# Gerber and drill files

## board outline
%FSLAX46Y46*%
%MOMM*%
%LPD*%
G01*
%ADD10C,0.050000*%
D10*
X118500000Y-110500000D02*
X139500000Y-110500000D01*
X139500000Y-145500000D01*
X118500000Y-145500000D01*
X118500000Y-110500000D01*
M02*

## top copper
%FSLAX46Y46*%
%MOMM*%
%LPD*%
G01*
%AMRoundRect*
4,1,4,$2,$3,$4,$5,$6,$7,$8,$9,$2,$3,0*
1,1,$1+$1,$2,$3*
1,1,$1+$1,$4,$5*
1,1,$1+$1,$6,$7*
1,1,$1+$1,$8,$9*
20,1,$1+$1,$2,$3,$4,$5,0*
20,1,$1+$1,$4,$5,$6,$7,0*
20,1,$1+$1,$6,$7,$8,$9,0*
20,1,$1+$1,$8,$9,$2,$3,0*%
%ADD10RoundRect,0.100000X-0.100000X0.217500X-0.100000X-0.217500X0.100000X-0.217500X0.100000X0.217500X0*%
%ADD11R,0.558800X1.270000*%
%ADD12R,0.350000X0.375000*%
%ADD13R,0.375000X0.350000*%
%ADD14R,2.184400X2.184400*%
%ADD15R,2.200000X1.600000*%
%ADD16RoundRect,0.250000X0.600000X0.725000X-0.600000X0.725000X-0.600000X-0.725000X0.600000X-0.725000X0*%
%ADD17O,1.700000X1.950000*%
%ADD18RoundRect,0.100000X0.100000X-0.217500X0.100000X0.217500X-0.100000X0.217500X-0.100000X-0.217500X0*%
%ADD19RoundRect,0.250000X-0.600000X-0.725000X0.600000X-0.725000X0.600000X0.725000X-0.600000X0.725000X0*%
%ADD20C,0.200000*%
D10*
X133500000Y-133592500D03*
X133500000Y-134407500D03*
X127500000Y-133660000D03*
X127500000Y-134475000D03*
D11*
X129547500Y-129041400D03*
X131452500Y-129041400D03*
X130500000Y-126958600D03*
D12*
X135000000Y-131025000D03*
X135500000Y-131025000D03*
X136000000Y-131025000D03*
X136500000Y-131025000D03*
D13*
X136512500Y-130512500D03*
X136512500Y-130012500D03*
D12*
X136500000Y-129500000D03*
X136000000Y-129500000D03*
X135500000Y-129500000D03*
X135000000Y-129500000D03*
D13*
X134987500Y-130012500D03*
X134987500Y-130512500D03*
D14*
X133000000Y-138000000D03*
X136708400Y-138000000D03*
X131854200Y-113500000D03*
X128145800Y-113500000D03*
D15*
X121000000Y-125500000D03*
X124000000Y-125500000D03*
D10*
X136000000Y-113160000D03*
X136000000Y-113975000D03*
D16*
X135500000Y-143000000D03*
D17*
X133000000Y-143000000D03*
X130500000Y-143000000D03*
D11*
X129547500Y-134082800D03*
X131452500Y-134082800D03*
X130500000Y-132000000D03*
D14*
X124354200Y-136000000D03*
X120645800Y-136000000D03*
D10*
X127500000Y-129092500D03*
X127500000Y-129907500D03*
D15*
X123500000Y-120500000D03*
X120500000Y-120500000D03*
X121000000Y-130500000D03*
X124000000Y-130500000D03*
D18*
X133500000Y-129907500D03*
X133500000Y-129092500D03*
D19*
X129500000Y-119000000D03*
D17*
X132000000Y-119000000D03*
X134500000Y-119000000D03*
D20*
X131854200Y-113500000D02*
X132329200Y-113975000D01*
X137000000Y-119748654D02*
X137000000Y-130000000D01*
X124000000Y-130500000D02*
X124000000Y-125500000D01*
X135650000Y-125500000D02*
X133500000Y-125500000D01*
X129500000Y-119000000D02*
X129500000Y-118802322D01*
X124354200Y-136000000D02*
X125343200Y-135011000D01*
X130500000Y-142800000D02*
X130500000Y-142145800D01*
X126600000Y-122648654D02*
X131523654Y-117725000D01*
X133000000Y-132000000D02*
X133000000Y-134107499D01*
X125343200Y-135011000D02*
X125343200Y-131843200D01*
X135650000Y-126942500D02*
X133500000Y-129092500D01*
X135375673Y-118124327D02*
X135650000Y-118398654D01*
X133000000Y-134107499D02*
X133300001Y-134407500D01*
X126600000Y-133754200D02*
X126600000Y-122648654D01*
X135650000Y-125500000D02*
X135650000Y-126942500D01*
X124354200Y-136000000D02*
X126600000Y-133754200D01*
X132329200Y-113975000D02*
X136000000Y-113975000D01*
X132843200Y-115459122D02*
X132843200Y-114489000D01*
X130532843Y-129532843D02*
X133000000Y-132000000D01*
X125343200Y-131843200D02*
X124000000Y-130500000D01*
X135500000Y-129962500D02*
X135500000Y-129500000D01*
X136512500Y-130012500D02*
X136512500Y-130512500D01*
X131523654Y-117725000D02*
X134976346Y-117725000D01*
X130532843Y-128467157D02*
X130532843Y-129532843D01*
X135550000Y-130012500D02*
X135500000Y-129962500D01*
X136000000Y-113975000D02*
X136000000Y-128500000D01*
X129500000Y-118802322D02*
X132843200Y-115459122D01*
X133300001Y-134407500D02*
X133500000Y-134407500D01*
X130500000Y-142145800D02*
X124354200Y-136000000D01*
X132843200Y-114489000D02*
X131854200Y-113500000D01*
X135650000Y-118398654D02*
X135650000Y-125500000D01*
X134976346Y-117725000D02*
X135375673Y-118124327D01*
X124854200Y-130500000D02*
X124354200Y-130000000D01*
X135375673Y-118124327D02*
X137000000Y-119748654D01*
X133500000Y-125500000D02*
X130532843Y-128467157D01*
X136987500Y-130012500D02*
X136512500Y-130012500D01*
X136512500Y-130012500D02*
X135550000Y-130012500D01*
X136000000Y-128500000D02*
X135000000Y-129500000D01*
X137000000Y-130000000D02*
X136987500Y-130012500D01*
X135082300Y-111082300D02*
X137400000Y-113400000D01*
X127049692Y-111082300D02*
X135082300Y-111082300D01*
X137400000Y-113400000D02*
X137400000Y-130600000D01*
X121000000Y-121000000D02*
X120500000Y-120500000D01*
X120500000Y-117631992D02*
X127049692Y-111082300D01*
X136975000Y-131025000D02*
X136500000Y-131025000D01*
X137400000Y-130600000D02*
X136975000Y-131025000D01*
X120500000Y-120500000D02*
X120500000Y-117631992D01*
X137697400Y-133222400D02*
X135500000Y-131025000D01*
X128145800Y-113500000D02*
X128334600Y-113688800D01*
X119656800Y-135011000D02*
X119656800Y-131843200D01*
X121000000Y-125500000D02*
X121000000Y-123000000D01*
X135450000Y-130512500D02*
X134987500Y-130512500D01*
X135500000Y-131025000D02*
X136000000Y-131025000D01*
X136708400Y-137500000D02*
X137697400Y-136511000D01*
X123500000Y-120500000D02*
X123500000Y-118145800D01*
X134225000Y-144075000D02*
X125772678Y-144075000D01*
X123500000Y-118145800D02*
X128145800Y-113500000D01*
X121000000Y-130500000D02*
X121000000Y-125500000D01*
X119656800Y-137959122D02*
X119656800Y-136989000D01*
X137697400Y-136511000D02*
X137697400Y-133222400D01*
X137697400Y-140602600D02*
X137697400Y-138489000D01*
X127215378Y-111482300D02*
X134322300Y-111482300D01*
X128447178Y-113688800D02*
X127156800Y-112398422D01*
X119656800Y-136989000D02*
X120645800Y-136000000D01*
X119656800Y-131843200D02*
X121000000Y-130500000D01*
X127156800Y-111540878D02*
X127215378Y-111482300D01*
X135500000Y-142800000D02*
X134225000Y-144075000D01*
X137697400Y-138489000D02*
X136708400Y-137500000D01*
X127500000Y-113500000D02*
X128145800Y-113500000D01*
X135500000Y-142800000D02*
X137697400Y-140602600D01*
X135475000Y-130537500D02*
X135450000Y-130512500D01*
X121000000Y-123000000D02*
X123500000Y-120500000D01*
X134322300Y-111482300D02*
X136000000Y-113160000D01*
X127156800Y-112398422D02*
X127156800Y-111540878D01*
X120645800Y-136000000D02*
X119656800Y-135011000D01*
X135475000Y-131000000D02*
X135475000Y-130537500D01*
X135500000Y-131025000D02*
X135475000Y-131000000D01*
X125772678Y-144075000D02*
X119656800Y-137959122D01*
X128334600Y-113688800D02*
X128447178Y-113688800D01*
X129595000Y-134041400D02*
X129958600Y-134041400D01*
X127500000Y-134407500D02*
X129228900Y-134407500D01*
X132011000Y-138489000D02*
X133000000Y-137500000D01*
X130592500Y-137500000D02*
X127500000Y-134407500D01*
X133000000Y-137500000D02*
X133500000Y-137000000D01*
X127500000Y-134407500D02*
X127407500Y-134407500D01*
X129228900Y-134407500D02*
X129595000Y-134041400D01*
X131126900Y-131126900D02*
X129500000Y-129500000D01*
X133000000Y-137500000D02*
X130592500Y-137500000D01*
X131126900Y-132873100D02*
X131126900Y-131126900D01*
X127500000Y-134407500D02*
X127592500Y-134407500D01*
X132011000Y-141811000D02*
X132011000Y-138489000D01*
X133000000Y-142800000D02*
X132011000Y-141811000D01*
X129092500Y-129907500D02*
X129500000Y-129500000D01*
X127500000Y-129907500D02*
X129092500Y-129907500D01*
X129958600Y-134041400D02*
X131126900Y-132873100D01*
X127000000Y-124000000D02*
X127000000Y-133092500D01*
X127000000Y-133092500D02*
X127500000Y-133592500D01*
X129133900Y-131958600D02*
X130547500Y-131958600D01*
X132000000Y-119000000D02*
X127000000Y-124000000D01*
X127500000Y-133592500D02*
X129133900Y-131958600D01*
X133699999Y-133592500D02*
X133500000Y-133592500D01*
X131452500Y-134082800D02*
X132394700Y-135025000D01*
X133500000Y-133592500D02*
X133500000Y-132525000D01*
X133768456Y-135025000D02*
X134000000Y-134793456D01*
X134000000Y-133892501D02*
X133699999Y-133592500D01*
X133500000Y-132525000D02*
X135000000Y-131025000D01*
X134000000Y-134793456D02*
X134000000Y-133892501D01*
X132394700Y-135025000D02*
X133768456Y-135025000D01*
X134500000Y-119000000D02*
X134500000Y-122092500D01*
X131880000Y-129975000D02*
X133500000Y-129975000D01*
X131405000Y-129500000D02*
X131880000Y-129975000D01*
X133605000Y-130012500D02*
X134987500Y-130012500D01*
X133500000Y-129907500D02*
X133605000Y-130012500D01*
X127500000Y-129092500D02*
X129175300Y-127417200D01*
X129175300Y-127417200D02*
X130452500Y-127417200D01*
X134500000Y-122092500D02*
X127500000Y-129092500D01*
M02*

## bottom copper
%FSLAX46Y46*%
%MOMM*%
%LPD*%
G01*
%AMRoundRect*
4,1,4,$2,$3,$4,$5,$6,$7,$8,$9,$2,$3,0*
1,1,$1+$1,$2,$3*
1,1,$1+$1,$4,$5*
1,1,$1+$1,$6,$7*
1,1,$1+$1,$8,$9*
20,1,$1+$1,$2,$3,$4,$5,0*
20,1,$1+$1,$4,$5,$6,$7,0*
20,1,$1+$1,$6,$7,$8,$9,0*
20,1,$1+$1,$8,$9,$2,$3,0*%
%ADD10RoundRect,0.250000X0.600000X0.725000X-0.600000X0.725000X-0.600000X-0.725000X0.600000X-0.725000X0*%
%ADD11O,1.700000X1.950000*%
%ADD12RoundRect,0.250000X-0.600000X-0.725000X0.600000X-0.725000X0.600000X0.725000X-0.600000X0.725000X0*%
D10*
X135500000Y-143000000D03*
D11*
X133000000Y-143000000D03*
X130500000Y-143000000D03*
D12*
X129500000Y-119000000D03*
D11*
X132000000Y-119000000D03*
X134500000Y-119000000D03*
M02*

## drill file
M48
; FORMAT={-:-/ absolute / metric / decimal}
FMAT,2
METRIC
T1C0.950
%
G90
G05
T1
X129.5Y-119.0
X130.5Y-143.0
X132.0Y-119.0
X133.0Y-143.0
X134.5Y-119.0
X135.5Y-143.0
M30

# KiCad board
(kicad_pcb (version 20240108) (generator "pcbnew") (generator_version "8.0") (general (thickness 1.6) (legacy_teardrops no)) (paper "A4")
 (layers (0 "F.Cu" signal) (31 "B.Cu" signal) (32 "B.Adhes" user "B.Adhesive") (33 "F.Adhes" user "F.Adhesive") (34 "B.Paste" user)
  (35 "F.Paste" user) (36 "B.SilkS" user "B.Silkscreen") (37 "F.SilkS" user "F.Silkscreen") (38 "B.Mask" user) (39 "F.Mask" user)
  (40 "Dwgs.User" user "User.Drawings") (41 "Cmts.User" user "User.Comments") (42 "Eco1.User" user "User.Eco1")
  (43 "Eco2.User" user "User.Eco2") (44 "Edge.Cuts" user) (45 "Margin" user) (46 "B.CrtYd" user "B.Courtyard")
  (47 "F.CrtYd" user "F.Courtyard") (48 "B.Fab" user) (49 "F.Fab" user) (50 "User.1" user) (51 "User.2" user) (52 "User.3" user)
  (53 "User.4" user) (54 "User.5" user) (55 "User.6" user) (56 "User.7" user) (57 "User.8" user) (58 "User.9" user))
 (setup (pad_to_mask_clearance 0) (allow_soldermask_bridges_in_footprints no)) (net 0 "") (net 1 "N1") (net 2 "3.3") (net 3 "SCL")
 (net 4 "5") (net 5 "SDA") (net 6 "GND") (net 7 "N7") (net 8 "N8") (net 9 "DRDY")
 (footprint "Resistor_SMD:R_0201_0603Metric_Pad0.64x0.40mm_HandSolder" (layer "F.Cu") (at 133.5 134 -90)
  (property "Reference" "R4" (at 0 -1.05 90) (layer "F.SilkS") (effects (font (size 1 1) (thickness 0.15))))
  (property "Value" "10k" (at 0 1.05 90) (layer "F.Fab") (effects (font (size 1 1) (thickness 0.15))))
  (pad "" smd roundrect (at -0.4325 0 270) (size 0.458 0.36) (layers "F.Paste") (roundrect_rratio 0.25))
  (pad "" smd roundrect (at 0.4325 0 270) (size 0.458 0.36) (layers "F.Paste") (roundrect_rratio 0.25))
  (pad "1" smd roundrect (at -0.4075 0 270) (size 0.635 0.4) (layers "F.Cu" "F.Mask") (roundrect_rratio 0.25) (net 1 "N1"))
  (pad "2" smd roundrect (at 0.4075 0 270) (size 0.635 0.4) (layers "F.Cu" "F.Mask") (roundrect_rratio 0.25) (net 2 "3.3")))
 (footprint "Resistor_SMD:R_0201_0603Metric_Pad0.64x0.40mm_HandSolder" (layer "F.Cu") (at 127.5 134.0675 -90)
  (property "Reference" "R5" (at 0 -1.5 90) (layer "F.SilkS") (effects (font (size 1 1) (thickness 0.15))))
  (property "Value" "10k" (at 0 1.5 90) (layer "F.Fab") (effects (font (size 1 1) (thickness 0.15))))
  (pad "" smd roundrect (at -0.4325 0 270) (size 0.458 0.36) (layers "F.Paste") (roundrect_rratio 0.25))
  (pad "" smd roundrect (at 0.4325 0 270) (size 0.458 0.36) (layers "F.Paste") (roundrect_rratio 0.25))
  (pad "1" smd roundrect (at -0.4075 0 270) (size 0.635 0.4) (layers "F.Cu" "F.Mask") (roundrect_rratio 0.25) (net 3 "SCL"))
  (pad "2" smd roundrect (at 0.4075 0 270) (size 0.635 0.4) (layers "F.Cu" "F.Mask") (roundrect_rratio 0.25) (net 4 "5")))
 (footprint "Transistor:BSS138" (layer "F.Cu") (at 130.5 128)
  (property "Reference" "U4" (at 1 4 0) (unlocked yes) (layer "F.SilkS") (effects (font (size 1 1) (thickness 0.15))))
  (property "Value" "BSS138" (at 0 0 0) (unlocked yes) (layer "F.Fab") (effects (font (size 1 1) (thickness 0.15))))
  (pad "1" smd rect (at -0.9525 1.0414) (size 0.5588 1.27) (layers "F.Cu" "F.Paste" "F.Mask") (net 4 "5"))
  (pad "2" smd rect (at 0.9525 1.0414) (size 0.5588 1.27) (layers "F.Cu" "F.Paste" "F.Mask") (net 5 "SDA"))
  (pad "3" smd rect (at 0 -1.0414) (size 0.5588 1.27) (layers "F.Cu" "F.Paste" "F.Mask") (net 5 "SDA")))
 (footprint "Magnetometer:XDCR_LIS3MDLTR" (layer "F.Cu") (at 135.75 130.2625 90)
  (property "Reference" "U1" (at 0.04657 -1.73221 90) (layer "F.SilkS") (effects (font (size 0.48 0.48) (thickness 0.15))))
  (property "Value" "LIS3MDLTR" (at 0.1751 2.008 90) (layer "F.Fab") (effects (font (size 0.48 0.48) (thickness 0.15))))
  (pad "1" smd rect (at -0.7625 -0.75 90) (size 0.375 0.35) (layers "F.Cu" "F.Paste") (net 1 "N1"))
  (pad "2" smd rect (at -0.7625 -0.25 90) (size 0.375 0.35) (layers "F.Cu" "F.Paste") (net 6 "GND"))
  (pad "3" smd rect (at -0.7625 0.25 90) (size 0.375 0.35) (layers "F.Cu" "F.Paste") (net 6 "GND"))
  (pad "4" smd rect (at -0.7625 0.75 90) (size 0.375 0.35) (layers "F.Cu" "F.Paste") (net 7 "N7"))
  (pad "5" smd rect (at -0.25 0.7625 90) (size 0.35 0.375) (layers "F.Cu" "F.Paste") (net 2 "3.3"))
  (pad "6" smd rect (at 0.25 0.7625 90) (size 0.35 0.375) (layers "F.Cu" "F.Paste") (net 2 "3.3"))
  (pad "7" smd rect (at 0.7625 0.75 90) (size 0.375 0.35) (layers "F.Cu" "F.Paste") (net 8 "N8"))
  (pad "8" smd rect (at 0.7625 0.25 90) (size 0.375 0.35) (layers "F.Cu" "F.Paste") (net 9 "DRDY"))
  (pad "9" smd rect (at 0.7625 -0.25 90) (size 0.375 0.35) (layers "F.Cu" "F.Paste") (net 2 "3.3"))
  (pad "10" smd rect (at 0.7625 -0.75 90) (size 0.375 0.35) (layers "F.Cu" "F.Paste") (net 2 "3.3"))
  (pad "11" smd rect (at 0.25 -0.7625 90) (size 0.35 0.375) (layers "F.Cu" "F.Paste") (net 5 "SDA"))
  (pad "12" smd rect (at -0.25 -0.7625 90) (size 0.35 0.375) (layers "F.Cu" "F.Paste") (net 6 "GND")))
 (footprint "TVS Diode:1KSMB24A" (layer "F.Cu") (at 134.8542 138)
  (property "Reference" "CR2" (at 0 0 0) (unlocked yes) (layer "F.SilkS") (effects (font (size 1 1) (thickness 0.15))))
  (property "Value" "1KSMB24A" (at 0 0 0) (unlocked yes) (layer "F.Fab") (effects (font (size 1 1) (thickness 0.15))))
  (pad "1" smd rect (at -1.8542 0 90) (size 2.1844 2.1844) (layers "F.Cu" "F.Paste" "F.Mask") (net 4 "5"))
  (pad "2" smd rect (at 1.8542 0 90) (size 2.1844 2.1844) (layers "F.Cu" "F.Paste" "F.Mask") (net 6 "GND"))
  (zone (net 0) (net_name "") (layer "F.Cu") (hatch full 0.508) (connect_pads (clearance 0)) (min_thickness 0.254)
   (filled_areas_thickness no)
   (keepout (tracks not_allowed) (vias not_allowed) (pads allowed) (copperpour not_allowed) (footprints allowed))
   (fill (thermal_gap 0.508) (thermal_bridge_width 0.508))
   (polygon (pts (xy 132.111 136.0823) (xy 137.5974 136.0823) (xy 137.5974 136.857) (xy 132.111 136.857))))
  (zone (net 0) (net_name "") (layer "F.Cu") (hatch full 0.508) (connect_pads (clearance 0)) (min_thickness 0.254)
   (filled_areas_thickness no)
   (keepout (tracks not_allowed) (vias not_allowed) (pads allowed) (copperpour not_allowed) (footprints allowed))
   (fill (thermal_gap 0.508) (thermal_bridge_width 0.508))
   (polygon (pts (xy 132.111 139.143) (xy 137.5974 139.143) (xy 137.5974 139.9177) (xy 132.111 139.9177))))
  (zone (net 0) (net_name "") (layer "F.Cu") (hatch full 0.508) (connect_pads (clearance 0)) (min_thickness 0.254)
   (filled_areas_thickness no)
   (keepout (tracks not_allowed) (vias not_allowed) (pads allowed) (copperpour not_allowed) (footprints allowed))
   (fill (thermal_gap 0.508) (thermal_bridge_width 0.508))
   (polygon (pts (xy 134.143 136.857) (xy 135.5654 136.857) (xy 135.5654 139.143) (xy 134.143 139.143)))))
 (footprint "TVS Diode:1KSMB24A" (layer "F.Cu") (at 130 113.5 180)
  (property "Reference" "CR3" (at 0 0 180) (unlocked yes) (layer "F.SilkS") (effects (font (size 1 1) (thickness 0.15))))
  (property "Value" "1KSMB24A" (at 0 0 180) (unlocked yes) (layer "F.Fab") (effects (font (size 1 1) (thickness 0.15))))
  (pad "1" smd rect (at -1.8542 0 270) (size 2.1844 2.1844) (layers "F.Cu" "F.Paste" "F.Mask") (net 2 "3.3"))
  (pad "2" smd rect (at 1.8542 0 270) (size 2.1844 2.1844) (layers "F.Cu" "F.Paste" "F.Mask") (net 6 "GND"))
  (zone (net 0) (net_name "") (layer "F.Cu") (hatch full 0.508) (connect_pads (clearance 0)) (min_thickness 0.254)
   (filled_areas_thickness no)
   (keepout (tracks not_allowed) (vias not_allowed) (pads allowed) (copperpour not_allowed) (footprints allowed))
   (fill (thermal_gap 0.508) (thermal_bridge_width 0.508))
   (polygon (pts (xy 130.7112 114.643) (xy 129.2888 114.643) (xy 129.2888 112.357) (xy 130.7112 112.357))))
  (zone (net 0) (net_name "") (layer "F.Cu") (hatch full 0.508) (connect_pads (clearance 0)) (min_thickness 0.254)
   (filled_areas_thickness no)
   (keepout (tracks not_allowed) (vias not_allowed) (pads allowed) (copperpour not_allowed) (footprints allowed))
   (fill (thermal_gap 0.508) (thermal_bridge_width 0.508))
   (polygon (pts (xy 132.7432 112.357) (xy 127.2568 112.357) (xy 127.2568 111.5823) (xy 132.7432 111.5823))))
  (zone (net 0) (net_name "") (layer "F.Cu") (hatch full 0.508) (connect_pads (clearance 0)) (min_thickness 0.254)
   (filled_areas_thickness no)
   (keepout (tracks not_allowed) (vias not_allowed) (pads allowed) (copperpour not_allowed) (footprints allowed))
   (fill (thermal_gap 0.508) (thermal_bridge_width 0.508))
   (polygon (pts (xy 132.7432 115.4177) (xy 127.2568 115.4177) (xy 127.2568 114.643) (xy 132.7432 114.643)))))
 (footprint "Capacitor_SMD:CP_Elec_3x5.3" (layer "F.Cu") (at 122.5 125.5)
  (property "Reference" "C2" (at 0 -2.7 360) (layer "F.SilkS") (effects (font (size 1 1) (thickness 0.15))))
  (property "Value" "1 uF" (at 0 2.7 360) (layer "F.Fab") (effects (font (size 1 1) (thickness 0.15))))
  (pad "1" smd rect (at -1.5 0) (size 2.2 1.6) (layers "F.Cu" "F.Paste" "F.Mask") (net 6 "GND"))
  (pad "2" smd rect (at 1.5 0) (size 2.2 1.6) (layers "F.Cu" "F.Paste" "F.Mask") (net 2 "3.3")))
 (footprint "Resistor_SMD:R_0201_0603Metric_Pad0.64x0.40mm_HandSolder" (layer "F.Cu") (at 136 113.5675 -90)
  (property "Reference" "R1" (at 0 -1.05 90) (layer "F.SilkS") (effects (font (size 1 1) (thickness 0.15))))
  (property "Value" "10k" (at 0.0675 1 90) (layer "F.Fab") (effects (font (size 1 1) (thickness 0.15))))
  (pad "" smd roundrect (at -0.4325 0 270) (size 0.458 0.36) (layers "F.Paste") (roundrect_rratio 0.25))
  (pad "" smd roundrect (at 0.4325 0 270) (size 0.458 0.36) (layers "F.Paste") (roundrect_rratio 0.25))
  (pad "1" smd roundrect (at -0.4075 0 270) (size 0.635 0.4) (layers "F.Cu" "F.Mask") (roundrect_rratio 0.25) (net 6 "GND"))
  (pad "2" smd roundrect (at 0.4075 0 270) (size 0.635 0.4) (layers "F.Cu" "F.Mask") (roundrect_rratio 0.25) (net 2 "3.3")))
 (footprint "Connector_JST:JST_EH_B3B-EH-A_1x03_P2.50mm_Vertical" (layer "F.Cu") (at 135.5 143 180)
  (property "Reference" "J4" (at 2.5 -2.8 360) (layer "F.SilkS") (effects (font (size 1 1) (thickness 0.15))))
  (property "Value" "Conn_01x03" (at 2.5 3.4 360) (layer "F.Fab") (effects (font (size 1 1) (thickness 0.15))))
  (pad "1" thru_hole roundrect (at 0 0 180) (size 1.7 1.95) (drill 0.95) (layers "*.Cu" "*.Mask") (remove_unused_layers no)
   (roundrect_rratio 0.147059) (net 6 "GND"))
  (pad "2" thru_hole oval (at 2.5 0 180) (size 1.7 1.95) (drill 0.95) (layers "*.Cu" "*.Mask") (remove_unused_layers no) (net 4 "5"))
  (pad "3" thru_hole oval (at 5 0 180) (size 1.7 1.95) (drill 0.95) (layers "*.Cu" "*.Mask") (remove_unused_layers no) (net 2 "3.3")))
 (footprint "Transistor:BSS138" (layer "F.Cu") (at 130.5 133.0414)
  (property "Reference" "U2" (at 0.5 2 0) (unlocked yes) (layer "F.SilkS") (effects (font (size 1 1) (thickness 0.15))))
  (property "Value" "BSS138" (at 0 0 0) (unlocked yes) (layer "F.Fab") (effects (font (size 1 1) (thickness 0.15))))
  (pad "1" smd rect (at -0.9525 1.0414) (size 0.5588 1.27) (layers "F.Cu" "F.Paste" "F.Mask") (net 4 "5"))
  (pad "2" smd rect (at 0.9525 1.0414) (size 0.5588 1.27) (layers "F.Cu" "F.Paste" "F.Mask") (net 1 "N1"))
  (pad "3" smd rect (at 0 -1.0414) (size 0.5588 1.27) (layers "F.Cu" "F.Paste" "F.Mask") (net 3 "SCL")))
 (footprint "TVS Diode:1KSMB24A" (layer "F.Cu") (at 122.5 136 180)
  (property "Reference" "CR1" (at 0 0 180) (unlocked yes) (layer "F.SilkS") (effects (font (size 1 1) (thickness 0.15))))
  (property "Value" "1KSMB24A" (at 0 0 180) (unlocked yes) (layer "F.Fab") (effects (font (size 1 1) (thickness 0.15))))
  (pad "1" smd rect (at -1.8542 0 270) (size 2.1844 2.1844) (layers "F.Cu" "F.Paste" "F.Mask") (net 2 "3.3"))
  (pad "2" smd rect (at 1.8542 0 270) (size 2.1844 2.1844) (layers "F.Cu" "F.Paste" "F.Mask") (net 6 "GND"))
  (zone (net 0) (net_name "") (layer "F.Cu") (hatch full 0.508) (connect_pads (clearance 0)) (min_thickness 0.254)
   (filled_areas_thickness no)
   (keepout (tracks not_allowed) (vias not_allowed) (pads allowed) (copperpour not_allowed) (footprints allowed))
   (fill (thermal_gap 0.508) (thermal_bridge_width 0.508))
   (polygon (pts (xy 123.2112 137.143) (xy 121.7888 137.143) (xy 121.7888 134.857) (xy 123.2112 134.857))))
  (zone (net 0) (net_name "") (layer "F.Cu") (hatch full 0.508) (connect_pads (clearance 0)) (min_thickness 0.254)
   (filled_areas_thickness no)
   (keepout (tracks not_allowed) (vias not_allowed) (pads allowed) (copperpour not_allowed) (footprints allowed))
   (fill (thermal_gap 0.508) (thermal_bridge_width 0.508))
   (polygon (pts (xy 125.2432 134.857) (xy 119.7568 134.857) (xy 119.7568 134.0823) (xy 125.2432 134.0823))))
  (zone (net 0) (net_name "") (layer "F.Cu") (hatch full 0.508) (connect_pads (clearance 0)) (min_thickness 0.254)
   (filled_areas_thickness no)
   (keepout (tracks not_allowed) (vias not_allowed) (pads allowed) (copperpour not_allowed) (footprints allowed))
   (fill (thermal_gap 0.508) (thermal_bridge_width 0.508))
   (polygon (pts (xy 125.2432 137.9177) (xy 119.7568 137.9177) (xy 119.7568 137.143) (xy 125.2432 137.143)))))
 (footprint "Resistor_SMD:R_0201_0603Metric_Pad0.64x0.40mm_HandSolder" (layer "F.Cu") (at 127.5 129.5 -90)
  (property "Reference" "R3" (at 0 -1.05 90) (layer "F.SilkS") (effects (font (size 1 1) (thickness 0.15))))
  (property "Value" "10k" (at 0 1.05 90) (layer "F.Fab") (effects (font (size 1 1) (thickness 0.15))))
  (pad "" smd roundrect (at -0.4325 0 270) (size 0.458 0.36) (layers "F.Paste") (roundrect_rratio 0.25))
  (pad "" smd roundrect (at 0.4325 0 270) (size 0.458 0.36) (layers "F.Paste") (roundrect_rratio 0.25))
  (pad "1" smd roundrect (at -0.4075 0 270) (size 0.635 0.4) (layers "F.Cu" "F.Mask") (roundrect_rratio 0.25) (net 5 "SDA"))
  (pad "2" smd roundrect (at 0.4075 0 270) (size 0.635 0.4) (layers "F.Cu" "F.Mask") (roundrect_rratio 0.25) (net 4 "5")))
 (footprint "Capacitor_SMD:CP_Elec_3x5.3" (layer "F.Cu") (at 122 120.5 180)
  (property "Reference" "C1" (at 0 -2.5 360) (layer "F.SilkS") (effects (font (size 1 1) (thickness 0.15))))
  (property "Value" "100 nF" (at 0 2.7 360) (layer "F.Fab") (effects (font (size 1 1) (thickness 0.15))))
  (pad "1" smd rect (at -1.5 0 180) (size 2.2 1.6) (layers "F.Cu" "F.Paste" "F.Mask") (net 6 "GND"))
  (pad "2" smd rect (at 1.5 0 180) (size 2.2 1.6) (layers "F.Cu" "F.Paste" "F.Mask") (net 7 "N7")))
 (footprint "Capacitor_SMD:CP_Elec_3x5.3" (layer "F.Cu") (at 122.5 130.5)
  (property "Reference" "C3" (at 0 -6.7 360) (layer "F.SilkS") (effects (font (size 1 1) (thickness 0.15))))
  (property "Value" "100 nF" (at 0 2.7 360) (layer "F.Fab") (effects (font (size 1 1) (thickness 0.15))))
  (pad "1" smd rect (at -1.5 0) (size 2.2 1.6) (layers "F.Cu" "F.Paste" "F.Mask") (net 6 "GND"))
  (pad "2" smd rect (at 1.5 0) (size 2.2 1.6) (layers "F.Cu" "F.Paste" "F.Mask") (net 2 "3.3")))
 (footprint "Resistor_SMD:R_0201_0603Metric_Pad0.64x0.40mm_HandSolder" (layer "F.Cu") (at 133.5 129.5 90)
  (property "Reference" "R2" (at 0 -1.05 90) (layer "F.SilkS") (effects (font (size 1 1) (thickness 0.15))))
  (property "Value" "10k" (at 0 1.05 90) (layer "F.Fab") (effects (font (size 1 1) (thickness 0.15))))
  (pad "" smd roundrect (at -0.4325 0 90) (size 0.458 0.36) (layers "F.Paste") (roundrect_rratio 0.25))
  (pad "" smd roundrect (at 0.4325 0 90) (size 0.458 0.36) (layers "F.Paste") (roundrect_rratio 0.25))
  (pad "1" smd roundrect (at -0.4075 0 90) (size 0.635 0.4) (layers "F.Cu" "F.Mask") (roundrect_rratio 0.25) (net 5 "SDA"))
  (pad "2" smd roundrect (at 0.4075 0 90) (size 0.635 0.4) (layers "F.Cu" "F.Mask") (roundrect_rratio 0.25) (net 2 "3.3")))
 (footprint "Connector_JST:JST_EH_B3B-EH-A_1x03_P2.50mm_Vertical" (layer "F.Cu") (at 129.5 119)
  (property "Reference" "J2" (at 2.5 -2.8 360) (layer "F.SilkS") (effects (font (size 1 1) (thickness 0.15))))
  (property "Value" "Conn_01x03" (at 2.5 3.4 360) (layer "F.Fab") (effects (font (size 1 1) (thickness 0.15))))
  (pad "1" thru_hole roundrect (at 0 0) (size 1.7 1.95) (drill 0.95) (layers "*.Cu" "*.Mask") (remove_unused_layers no)
   (roundrect_rratio 0.147059) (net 2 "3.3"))
  (pad "2" thru_hole oval (at 2.5 0) (size 1.7 1.95) (drill 0.95) (layers "*.Cu" "*.Mask") (remove_unused_layers no) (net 3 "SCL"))
  (pad "3" thru_hole oval (at 5 0) (size 1.7 1.95) (drill 0.95) (layers "*.Cu" "*.Mask") (remove_unused_layers no) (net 5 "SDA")))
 (gr_rect (start 118.5 110.5) (end 139.5 145.5) (stroke (width 0.05) (type default)) (fill none) (layer "Edge.Cuts"))
 (segment (start 131.8542 113.5) (end 132.3292 113.975) (width 0.2) (layer "F.Cu") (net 2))
 (segment (start 137 119.748654) (end 137 130) (width 0.2) (layer "F.Cu") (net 2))
 (segment (start 124 130.5) (end 124 125.5) (width 0.2) (layer "F.Cu") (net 2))
 (segment (start 135.65 125.5) (end 133.5 125.5) (width 0.2) (layer "F.Cu") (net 2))
 (segment (start 129.5 119) (end 129.5 118.802322) (width 0.2) (layer "F.Cu") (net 2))
 (segment (start 124.3542 136) (end 125.3432 135.011) (width 0.2) (layer "F.Cu") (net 2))
 (segment (start 130.5 142.8) (end 130.5 142.1458) (width 0.2) (layer "F.Cu") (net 2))
 (segment (start 126.6 122.648654) (end 131.523654 117.725) (width 0.2) (layer "F.Cu") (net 2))
 (segment (start 133 132) (end 133 134.107499) (width 0.2) (layer "F.Cu") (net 2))
 (segment (start 125.3432 135.011) (end 125.3432 131.8432) (width 0.2) (layer "F.Cu") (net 2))
 (segment (start 135.65 126.9425) (end 133.5 129.0925) (width 0.2) (layer "F.Cu") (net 2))
 (segment (start 135.375673 118.124327) (end 135.65 118.398654) (width 0.2) (layer "F.Cu") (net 2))
 (segment (start 133 134.107499) (end 133.300001 134.4075) (width 0.2) (layer "F.Cu") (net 2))
 (segment (start 126.6 133.7542) (end 126.6 122.648654) (width 0.2) (layer "F.Cu") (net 2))
 (segment (start 135.65 125.5) (end 135.65 126.9425) (width 0.2) (layer "F.Cu") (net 2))
 (segment (start 124.3542 136) (end 126.6 133.7542) (width 0.2) (layer "F.Cu") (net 2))
 (segment (start 132.3292 113.975) (end 136 113.975) (width 0.2) (layer "F.Cu") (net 2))
 (segment (start 132.8432 115.459122) (end 132.8432 114.489) (width 0.2) (layer "F.Cu") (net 2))
 (segment (start 130.532843 129.532843) (end 133 132) (width 0.2) (layer "F.Cu") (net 2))
 (segment (start 125.3432 131.8432) (end 124 130.5) (width 0.2) (layer "F.Cu") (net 2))
 (segment (start 135.5 129.9625) (end 135.5 129.5) (width 0.2) (layer "F.Cu") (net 2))
 (segment (start 136.5125 130.0125) (end 136.5125 130.5125) (width 0.2) (layer "F.Cu") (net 2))
 (segment (start 131.523654 117.725) (end 134.976346 117.725) (width 0.2) (layer "F.Cu") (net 2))
 (segment (start 130.532843 128.467157) (end 130.532843 129.532843) (width 0.2) (layer "F.Cu") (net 2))
 (segment (start 135.55 130.0125) (end 135.5 129.9625) (width 0.2) (layer "F.Cu") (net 2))
 (segment (start 136 113.975) (end 136 128.5) (width 0.2) (layer "F.Cu") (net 2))
 (segment (start 129.5 118.802322) (end 132.8432 115.459122) (width 0.2) (layer "F.Cu") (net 2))
 (segment (start 133.300001 134.4075) (end 133.5 134.4075) (width 0.2) (layer "F.Cu") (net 2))
 (segment (start 130.5 142.1458) (end 124.3542 136) (width 0.2) (layer "F.Cu") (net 2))
 (segment (start 132.8432 114.489) (end 131.8542 113.5) (width 0.2) (layer "F.Cu") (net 2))
 (segment (start 135.65 118.398654) (end 135.65 125.5) (width 0.2) (layer "F.Cu") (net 2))
 (segment (start 134.976346 117.725) (end 135.375673 118.124327) (width 0.2) (layer "F.Cu") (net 2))
 (segment (start 124.8542 130.5) (end 124.3542 130) (width 0.2) (layer "F.Cu") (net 2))
 (segment (start 135.375673 118.124327) (end 137 119.748654) (width 0.2) (layer "F.Cu") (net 2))
 (segment (start 133.5 125.5) (end 130.532843 128.467157) (width 0.2) (layer "F.Cu") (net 2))
 (segment (start 136.9875 130.0125) (end 136.5125 130.0125) (width 0.2) (layer "F.Cu") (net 2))
 (segment (start 136.5125 130.0125) (end 135.55 130.0125) (width 0.2) (layer "F.Cu") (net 2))
 (segment (start 136 128.5) (end 135 129.5) (width 0.2) (layer "F.Cu") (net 2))
 (segment (start 137 130) (end 136.9875 130.0125) (width 0.2) (layer "F.Cu") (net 2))
 (segment (start 135.0823 111.0823) (end 137.4 113.4) (width 0.2) (layer "F.Cu") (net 7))
 (segment (start 127.049692 111.0823) (end 135.0823 111.0823) (width 0.2) (layer "F.Cu") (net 7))
 (segment (start 137.4 113.4) (end 137.4 130.6) (width 0.2) (layer "F.Cu") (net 7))
 (segment (start 121 121) (end 120.5 120.5) (width 0.2) (layer "F.Cu") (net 7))
 (segment (start 120.5 117.631992) (end 127.049692 111.0823) (width 0.2) (layer "F.Cu") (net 7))
 (segment (start 136.975 131.025) (end 136.5 131.025) (width 0.2) (layer "F.Cu") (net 7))
 (segment (start 137.4 130.6) (end 136.975 131.025) (width 0.2) (layer "F.Cu") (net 7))
 (segment (start 120.5 120.5) (end 120.5 117.631992) (width 0.2) (layer "F.Cu") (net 7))
 (segment (start 137.6974 133.2224) (end 135.5 131.025) (width 0.2) (layer "F.Cu") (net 6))
 (segment (start 128.1458 113.5) (end 128.3346 113.6888) (width 0.2) (layer "F.Cu") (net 6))
 (segment (start 119.6568 135.011) (end 119.6568 131.8432) (width 0.2) (layer "F.Cu") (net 6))
 (segment (start 121 125.5) (end 121 123) (width 0.2) (layer "F.Cu") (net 6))
 (segment (start 135.45 130.5125) (end 134.9875 130.5125) (width 0.2) (layer "F.Cu") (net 6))
 (segment (start 135.5 131.025) (end 136 131.025) (width 0.2) (layer "F.Cu") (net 6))
 (segment (start 136.7084 137.5) (end 137.6974 136.511) (width 0.2) (layer "F.Cu") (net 6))
 (segment (start 123.5 120.5) (end 123.5 118.1458) (width 0.2) (layer "F.Cu") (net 6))
 (segment (start 134.225 144.075) (end 125.772678 144.075) (width 0.2) (layer "F.Cu") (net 6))
 (segment (start 123.5 118.1458) (end 128.1458 113.5) (width 0.2) (layer "F.Cu") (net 6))
 (segment (start 121 130.5) (end 121 125.5) (width 0.2) (layer "F.Cu") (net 6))
 (segment (start 119.6568 137.959122) (end 119.6568 136.989) (width 0.2) (layer "F.Cu") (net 6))
 (segment (start 137.6974 136.511) (end 137.6974 133.2224) (width 0.2) (layer "F.Cu") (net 6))
 (segment (start 137.6974 140.6026) (end 137.6974 138.489) (width 0.2) (layer "F.Cu") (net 6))
 (segment (start 127.215378 111.4823) (end 134.3223 111.4823) (width 0.2) (layer "F.Cu") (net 6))
 (segment (start 128.447178 113.6888) (end 127.1568 112.398422) (width 0.2) (layer "F.Cu") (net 6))
 (segment (start 119.6568 136.989) (end 120.6458 136) (width 0.2) (layer "F.Cu") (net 6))
 (segment (start 119.6568 131.8432) (end 121 130.5) (width 0.2) (layer "F.Cu") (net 6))
 (segment (start 127.1568 111.540878) (end 127.215378 111.4823) (width 0.2) (layer "F.Cu") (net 6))
 (segment (start 135.5 142.8) (end 134.225 144.075) (width 0.2) (layer "F.Cu") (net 6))
 (segment (start 137.6974 138.489) (end 136.7084 137.5) (width 0.2) (layer "F.Cu") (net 6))
 (segment (start 127.5 113.5) (end 128.1458 113.5) (width 0.2) (layer "F.Cu") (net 6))
 (segment (start 135.5 142.8) (end 137.6974 140.6026) (width 0.2) (layer "F.Cu") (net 6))
 (segment (start 135.475 130.5375) (end 135.45 130.5125) (width 0.2) (layer "F.Cu") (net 6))
 (segment (start 121 123) (end 123.5 120.5) (width 0.2) (layer "F.Cu") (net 6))
 (segment (start 134.3223 111.4823) (end 136 113.16) (width 0.2) (layer "F.Cu") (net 6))
 (segment (start 127.1568 112.398422) (end 127.1568 111.540878) (width 0.2) (layer "F.Cu") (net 6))
 (segment (start 120.6458 136) (end 119.6568 135.011) (width 0.2) (layer "F.Cu") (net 6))
 (segment (start 135.475 131) (end 135.475 130.5375) (width 0.2) (layer "F.Cu") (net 6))
 (segment (start 135.5 131.025) (end 135.475 131) (width 0.2) (layer "F.Cu") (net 6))
 (segment (start 125.772678 144.075) (end 119.6568 137.959122) (width 0.2) (layer "F.Cu") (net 6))
 (segment (start 128.3346 113.6888) (end 128.447178 113.6888) (width 0.2) (layer "F.Cu") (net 6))
 (segment (start 129.595 134.0414) (end 129.9586 134.0414) (width 0.2) (layer "F.Cu") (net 4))
 (segment (start 127.5 134.4075) (end 129.2289 134.4075) (width 0.2) (layer "F.Cu") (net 4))
 (segment (start 132.011 138.489) (end 133 137.5) (width 0.2) (layer "F.Cu") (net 4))
 (segment (start 130.5925 137.5) (end 127.5 134.4075) (width 0.2) (layer "F.Cu") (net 4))
 (segment (start 133 137.5) (end 133.5 137) (width 0.2) (layer "F.Cu") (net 4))
 (segment (start 127.5 134.4075) (end 127.4075 134.4075) (width 0.2) (layer "F.Cu") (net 4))
 (segment (start 129.2289 134.4075) (end 129.595 134.0414) (width 0.2) (layer "F.Cu") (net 4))
 (segment (start 131.1269 131.1269) (end 129.5 129.5) (width 0.2) (layer "F.Cu") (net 4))
 (segment (start 133 137.5) (end 130.5925 137.5) (width 0.2) (layer "F.Cu") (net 4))
 (segment (start 131.1269 132.8731) (end 131.1269 131.1269) (width 0.2) (layer "F.Cu") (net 4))
 (segment (start 127.5 134.4075) (end 127.5925 134.4075) (width 0.2) (layer "F.Cu") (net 4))
 (segment (start 132.011 141.811) (end 132.011 138.489) (width 0.2) (layer "F.Cu") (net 4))
 (segment (start 133 142.8) (end 132.011 141.811) (width 0.2) (layer "F.Cu") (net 4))
 (segment (start 129.0925 129.9075) (end 129.5 129.5) (width 0.2) (layer "F.Cu") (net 4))
 (segment (start 127.5 129.9075) (end 129.0925 129.9075) (width 0.2) (layer "F.Cu") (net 4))
 (segment (start 129.9586 134.0414) (end 131.1269 132.8731) (width 0.2) (layer "F.Cu") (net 4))
 (segment (start 127 124) (end 127 133.0925) (width 0.2) (layer "F.Cu") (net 3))
 (segment (start 127 133.0925) (end 127.5 133.5925) (width 0.2) (layer "F.Cu") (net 3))
 (segment (start 129.1339 131.9586) (end 130.5475 131.9586) (width 0.2) (layer "F.Cu") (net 3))
 (segment (start 132 119) (end 127 124) (width 0.2) (layer "F.Cu") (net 3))
 (segment (start 127.5 133.5925) (end 129.1339 131.9586) (width 0.2) (layer "F.Cu") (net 3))
 (segment (start 133.699999 133.5925) (end 133.5 133.5925) (width 0.2) (layer "F.Cu") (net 1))
 (segment (start 131.4525 134.0828) (end 132.3947 135.025) (width 0.2) (layer "F.Cu") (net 1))
 (segment (start 133.5 133.5925) (end 133.5 132.525) (width 0.2) (layer "F.Cu") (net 1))
 (segment (start 133.768456 135.025) (end 134 134.793456) (width 0.2) (layer "F.Cu") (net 1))
 (segment (start 134 133.892501) (end 133.699999 133.5925) (width 0.2) (layer "F.Cu") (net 1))
 (segment (start 133.5 132.525) (end 135 131.025) (width 0.2) (layer "F.Cu") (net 1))
 (segment (start 134 134.793456) (end 134 133.892501) (width 0.2) (layer "F.Cu") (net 1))
 (segment (start 132.3947 135.025) (end 133.768456 135.025) (width 0.2) (layer "F.Cu") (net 1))
 (segment (start 134.5 119) (end 134.5 122.0925) (width 0.2) (layer "F.Cu") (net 5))
 (segment (start 131.88 129.975) (end 133.5 129.975) (width 0.2) (layer "F.Cu") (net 5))
 (segment (start 131.405 129.5) (end 131.88 129.975) (width 0.2) (layer "F.Cu") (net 5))
 (segment (start 133.605 130.0125) (end 134.9875 130.0125) (width 0.2) (layer "F.Cu") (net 5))
 (segment (start 133.5 129.9075) (end 133.605 130.0125) (width 0.2) (layer "F.Cu") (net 5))
 (segment (start 127.5 129.0925) (end 129.1753 127.4172) (width 0.2) (layer "F.Cu") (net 5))
 (segment (start 129.1753 127.4172) (end 130.4525 127.4172) (width 0.2) (layer "F.Cu") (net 5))
 (segment (start 134.5 122.0925) (end 127.5 129.0925) (width 0.2) (layer "F.Cu") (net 5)))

